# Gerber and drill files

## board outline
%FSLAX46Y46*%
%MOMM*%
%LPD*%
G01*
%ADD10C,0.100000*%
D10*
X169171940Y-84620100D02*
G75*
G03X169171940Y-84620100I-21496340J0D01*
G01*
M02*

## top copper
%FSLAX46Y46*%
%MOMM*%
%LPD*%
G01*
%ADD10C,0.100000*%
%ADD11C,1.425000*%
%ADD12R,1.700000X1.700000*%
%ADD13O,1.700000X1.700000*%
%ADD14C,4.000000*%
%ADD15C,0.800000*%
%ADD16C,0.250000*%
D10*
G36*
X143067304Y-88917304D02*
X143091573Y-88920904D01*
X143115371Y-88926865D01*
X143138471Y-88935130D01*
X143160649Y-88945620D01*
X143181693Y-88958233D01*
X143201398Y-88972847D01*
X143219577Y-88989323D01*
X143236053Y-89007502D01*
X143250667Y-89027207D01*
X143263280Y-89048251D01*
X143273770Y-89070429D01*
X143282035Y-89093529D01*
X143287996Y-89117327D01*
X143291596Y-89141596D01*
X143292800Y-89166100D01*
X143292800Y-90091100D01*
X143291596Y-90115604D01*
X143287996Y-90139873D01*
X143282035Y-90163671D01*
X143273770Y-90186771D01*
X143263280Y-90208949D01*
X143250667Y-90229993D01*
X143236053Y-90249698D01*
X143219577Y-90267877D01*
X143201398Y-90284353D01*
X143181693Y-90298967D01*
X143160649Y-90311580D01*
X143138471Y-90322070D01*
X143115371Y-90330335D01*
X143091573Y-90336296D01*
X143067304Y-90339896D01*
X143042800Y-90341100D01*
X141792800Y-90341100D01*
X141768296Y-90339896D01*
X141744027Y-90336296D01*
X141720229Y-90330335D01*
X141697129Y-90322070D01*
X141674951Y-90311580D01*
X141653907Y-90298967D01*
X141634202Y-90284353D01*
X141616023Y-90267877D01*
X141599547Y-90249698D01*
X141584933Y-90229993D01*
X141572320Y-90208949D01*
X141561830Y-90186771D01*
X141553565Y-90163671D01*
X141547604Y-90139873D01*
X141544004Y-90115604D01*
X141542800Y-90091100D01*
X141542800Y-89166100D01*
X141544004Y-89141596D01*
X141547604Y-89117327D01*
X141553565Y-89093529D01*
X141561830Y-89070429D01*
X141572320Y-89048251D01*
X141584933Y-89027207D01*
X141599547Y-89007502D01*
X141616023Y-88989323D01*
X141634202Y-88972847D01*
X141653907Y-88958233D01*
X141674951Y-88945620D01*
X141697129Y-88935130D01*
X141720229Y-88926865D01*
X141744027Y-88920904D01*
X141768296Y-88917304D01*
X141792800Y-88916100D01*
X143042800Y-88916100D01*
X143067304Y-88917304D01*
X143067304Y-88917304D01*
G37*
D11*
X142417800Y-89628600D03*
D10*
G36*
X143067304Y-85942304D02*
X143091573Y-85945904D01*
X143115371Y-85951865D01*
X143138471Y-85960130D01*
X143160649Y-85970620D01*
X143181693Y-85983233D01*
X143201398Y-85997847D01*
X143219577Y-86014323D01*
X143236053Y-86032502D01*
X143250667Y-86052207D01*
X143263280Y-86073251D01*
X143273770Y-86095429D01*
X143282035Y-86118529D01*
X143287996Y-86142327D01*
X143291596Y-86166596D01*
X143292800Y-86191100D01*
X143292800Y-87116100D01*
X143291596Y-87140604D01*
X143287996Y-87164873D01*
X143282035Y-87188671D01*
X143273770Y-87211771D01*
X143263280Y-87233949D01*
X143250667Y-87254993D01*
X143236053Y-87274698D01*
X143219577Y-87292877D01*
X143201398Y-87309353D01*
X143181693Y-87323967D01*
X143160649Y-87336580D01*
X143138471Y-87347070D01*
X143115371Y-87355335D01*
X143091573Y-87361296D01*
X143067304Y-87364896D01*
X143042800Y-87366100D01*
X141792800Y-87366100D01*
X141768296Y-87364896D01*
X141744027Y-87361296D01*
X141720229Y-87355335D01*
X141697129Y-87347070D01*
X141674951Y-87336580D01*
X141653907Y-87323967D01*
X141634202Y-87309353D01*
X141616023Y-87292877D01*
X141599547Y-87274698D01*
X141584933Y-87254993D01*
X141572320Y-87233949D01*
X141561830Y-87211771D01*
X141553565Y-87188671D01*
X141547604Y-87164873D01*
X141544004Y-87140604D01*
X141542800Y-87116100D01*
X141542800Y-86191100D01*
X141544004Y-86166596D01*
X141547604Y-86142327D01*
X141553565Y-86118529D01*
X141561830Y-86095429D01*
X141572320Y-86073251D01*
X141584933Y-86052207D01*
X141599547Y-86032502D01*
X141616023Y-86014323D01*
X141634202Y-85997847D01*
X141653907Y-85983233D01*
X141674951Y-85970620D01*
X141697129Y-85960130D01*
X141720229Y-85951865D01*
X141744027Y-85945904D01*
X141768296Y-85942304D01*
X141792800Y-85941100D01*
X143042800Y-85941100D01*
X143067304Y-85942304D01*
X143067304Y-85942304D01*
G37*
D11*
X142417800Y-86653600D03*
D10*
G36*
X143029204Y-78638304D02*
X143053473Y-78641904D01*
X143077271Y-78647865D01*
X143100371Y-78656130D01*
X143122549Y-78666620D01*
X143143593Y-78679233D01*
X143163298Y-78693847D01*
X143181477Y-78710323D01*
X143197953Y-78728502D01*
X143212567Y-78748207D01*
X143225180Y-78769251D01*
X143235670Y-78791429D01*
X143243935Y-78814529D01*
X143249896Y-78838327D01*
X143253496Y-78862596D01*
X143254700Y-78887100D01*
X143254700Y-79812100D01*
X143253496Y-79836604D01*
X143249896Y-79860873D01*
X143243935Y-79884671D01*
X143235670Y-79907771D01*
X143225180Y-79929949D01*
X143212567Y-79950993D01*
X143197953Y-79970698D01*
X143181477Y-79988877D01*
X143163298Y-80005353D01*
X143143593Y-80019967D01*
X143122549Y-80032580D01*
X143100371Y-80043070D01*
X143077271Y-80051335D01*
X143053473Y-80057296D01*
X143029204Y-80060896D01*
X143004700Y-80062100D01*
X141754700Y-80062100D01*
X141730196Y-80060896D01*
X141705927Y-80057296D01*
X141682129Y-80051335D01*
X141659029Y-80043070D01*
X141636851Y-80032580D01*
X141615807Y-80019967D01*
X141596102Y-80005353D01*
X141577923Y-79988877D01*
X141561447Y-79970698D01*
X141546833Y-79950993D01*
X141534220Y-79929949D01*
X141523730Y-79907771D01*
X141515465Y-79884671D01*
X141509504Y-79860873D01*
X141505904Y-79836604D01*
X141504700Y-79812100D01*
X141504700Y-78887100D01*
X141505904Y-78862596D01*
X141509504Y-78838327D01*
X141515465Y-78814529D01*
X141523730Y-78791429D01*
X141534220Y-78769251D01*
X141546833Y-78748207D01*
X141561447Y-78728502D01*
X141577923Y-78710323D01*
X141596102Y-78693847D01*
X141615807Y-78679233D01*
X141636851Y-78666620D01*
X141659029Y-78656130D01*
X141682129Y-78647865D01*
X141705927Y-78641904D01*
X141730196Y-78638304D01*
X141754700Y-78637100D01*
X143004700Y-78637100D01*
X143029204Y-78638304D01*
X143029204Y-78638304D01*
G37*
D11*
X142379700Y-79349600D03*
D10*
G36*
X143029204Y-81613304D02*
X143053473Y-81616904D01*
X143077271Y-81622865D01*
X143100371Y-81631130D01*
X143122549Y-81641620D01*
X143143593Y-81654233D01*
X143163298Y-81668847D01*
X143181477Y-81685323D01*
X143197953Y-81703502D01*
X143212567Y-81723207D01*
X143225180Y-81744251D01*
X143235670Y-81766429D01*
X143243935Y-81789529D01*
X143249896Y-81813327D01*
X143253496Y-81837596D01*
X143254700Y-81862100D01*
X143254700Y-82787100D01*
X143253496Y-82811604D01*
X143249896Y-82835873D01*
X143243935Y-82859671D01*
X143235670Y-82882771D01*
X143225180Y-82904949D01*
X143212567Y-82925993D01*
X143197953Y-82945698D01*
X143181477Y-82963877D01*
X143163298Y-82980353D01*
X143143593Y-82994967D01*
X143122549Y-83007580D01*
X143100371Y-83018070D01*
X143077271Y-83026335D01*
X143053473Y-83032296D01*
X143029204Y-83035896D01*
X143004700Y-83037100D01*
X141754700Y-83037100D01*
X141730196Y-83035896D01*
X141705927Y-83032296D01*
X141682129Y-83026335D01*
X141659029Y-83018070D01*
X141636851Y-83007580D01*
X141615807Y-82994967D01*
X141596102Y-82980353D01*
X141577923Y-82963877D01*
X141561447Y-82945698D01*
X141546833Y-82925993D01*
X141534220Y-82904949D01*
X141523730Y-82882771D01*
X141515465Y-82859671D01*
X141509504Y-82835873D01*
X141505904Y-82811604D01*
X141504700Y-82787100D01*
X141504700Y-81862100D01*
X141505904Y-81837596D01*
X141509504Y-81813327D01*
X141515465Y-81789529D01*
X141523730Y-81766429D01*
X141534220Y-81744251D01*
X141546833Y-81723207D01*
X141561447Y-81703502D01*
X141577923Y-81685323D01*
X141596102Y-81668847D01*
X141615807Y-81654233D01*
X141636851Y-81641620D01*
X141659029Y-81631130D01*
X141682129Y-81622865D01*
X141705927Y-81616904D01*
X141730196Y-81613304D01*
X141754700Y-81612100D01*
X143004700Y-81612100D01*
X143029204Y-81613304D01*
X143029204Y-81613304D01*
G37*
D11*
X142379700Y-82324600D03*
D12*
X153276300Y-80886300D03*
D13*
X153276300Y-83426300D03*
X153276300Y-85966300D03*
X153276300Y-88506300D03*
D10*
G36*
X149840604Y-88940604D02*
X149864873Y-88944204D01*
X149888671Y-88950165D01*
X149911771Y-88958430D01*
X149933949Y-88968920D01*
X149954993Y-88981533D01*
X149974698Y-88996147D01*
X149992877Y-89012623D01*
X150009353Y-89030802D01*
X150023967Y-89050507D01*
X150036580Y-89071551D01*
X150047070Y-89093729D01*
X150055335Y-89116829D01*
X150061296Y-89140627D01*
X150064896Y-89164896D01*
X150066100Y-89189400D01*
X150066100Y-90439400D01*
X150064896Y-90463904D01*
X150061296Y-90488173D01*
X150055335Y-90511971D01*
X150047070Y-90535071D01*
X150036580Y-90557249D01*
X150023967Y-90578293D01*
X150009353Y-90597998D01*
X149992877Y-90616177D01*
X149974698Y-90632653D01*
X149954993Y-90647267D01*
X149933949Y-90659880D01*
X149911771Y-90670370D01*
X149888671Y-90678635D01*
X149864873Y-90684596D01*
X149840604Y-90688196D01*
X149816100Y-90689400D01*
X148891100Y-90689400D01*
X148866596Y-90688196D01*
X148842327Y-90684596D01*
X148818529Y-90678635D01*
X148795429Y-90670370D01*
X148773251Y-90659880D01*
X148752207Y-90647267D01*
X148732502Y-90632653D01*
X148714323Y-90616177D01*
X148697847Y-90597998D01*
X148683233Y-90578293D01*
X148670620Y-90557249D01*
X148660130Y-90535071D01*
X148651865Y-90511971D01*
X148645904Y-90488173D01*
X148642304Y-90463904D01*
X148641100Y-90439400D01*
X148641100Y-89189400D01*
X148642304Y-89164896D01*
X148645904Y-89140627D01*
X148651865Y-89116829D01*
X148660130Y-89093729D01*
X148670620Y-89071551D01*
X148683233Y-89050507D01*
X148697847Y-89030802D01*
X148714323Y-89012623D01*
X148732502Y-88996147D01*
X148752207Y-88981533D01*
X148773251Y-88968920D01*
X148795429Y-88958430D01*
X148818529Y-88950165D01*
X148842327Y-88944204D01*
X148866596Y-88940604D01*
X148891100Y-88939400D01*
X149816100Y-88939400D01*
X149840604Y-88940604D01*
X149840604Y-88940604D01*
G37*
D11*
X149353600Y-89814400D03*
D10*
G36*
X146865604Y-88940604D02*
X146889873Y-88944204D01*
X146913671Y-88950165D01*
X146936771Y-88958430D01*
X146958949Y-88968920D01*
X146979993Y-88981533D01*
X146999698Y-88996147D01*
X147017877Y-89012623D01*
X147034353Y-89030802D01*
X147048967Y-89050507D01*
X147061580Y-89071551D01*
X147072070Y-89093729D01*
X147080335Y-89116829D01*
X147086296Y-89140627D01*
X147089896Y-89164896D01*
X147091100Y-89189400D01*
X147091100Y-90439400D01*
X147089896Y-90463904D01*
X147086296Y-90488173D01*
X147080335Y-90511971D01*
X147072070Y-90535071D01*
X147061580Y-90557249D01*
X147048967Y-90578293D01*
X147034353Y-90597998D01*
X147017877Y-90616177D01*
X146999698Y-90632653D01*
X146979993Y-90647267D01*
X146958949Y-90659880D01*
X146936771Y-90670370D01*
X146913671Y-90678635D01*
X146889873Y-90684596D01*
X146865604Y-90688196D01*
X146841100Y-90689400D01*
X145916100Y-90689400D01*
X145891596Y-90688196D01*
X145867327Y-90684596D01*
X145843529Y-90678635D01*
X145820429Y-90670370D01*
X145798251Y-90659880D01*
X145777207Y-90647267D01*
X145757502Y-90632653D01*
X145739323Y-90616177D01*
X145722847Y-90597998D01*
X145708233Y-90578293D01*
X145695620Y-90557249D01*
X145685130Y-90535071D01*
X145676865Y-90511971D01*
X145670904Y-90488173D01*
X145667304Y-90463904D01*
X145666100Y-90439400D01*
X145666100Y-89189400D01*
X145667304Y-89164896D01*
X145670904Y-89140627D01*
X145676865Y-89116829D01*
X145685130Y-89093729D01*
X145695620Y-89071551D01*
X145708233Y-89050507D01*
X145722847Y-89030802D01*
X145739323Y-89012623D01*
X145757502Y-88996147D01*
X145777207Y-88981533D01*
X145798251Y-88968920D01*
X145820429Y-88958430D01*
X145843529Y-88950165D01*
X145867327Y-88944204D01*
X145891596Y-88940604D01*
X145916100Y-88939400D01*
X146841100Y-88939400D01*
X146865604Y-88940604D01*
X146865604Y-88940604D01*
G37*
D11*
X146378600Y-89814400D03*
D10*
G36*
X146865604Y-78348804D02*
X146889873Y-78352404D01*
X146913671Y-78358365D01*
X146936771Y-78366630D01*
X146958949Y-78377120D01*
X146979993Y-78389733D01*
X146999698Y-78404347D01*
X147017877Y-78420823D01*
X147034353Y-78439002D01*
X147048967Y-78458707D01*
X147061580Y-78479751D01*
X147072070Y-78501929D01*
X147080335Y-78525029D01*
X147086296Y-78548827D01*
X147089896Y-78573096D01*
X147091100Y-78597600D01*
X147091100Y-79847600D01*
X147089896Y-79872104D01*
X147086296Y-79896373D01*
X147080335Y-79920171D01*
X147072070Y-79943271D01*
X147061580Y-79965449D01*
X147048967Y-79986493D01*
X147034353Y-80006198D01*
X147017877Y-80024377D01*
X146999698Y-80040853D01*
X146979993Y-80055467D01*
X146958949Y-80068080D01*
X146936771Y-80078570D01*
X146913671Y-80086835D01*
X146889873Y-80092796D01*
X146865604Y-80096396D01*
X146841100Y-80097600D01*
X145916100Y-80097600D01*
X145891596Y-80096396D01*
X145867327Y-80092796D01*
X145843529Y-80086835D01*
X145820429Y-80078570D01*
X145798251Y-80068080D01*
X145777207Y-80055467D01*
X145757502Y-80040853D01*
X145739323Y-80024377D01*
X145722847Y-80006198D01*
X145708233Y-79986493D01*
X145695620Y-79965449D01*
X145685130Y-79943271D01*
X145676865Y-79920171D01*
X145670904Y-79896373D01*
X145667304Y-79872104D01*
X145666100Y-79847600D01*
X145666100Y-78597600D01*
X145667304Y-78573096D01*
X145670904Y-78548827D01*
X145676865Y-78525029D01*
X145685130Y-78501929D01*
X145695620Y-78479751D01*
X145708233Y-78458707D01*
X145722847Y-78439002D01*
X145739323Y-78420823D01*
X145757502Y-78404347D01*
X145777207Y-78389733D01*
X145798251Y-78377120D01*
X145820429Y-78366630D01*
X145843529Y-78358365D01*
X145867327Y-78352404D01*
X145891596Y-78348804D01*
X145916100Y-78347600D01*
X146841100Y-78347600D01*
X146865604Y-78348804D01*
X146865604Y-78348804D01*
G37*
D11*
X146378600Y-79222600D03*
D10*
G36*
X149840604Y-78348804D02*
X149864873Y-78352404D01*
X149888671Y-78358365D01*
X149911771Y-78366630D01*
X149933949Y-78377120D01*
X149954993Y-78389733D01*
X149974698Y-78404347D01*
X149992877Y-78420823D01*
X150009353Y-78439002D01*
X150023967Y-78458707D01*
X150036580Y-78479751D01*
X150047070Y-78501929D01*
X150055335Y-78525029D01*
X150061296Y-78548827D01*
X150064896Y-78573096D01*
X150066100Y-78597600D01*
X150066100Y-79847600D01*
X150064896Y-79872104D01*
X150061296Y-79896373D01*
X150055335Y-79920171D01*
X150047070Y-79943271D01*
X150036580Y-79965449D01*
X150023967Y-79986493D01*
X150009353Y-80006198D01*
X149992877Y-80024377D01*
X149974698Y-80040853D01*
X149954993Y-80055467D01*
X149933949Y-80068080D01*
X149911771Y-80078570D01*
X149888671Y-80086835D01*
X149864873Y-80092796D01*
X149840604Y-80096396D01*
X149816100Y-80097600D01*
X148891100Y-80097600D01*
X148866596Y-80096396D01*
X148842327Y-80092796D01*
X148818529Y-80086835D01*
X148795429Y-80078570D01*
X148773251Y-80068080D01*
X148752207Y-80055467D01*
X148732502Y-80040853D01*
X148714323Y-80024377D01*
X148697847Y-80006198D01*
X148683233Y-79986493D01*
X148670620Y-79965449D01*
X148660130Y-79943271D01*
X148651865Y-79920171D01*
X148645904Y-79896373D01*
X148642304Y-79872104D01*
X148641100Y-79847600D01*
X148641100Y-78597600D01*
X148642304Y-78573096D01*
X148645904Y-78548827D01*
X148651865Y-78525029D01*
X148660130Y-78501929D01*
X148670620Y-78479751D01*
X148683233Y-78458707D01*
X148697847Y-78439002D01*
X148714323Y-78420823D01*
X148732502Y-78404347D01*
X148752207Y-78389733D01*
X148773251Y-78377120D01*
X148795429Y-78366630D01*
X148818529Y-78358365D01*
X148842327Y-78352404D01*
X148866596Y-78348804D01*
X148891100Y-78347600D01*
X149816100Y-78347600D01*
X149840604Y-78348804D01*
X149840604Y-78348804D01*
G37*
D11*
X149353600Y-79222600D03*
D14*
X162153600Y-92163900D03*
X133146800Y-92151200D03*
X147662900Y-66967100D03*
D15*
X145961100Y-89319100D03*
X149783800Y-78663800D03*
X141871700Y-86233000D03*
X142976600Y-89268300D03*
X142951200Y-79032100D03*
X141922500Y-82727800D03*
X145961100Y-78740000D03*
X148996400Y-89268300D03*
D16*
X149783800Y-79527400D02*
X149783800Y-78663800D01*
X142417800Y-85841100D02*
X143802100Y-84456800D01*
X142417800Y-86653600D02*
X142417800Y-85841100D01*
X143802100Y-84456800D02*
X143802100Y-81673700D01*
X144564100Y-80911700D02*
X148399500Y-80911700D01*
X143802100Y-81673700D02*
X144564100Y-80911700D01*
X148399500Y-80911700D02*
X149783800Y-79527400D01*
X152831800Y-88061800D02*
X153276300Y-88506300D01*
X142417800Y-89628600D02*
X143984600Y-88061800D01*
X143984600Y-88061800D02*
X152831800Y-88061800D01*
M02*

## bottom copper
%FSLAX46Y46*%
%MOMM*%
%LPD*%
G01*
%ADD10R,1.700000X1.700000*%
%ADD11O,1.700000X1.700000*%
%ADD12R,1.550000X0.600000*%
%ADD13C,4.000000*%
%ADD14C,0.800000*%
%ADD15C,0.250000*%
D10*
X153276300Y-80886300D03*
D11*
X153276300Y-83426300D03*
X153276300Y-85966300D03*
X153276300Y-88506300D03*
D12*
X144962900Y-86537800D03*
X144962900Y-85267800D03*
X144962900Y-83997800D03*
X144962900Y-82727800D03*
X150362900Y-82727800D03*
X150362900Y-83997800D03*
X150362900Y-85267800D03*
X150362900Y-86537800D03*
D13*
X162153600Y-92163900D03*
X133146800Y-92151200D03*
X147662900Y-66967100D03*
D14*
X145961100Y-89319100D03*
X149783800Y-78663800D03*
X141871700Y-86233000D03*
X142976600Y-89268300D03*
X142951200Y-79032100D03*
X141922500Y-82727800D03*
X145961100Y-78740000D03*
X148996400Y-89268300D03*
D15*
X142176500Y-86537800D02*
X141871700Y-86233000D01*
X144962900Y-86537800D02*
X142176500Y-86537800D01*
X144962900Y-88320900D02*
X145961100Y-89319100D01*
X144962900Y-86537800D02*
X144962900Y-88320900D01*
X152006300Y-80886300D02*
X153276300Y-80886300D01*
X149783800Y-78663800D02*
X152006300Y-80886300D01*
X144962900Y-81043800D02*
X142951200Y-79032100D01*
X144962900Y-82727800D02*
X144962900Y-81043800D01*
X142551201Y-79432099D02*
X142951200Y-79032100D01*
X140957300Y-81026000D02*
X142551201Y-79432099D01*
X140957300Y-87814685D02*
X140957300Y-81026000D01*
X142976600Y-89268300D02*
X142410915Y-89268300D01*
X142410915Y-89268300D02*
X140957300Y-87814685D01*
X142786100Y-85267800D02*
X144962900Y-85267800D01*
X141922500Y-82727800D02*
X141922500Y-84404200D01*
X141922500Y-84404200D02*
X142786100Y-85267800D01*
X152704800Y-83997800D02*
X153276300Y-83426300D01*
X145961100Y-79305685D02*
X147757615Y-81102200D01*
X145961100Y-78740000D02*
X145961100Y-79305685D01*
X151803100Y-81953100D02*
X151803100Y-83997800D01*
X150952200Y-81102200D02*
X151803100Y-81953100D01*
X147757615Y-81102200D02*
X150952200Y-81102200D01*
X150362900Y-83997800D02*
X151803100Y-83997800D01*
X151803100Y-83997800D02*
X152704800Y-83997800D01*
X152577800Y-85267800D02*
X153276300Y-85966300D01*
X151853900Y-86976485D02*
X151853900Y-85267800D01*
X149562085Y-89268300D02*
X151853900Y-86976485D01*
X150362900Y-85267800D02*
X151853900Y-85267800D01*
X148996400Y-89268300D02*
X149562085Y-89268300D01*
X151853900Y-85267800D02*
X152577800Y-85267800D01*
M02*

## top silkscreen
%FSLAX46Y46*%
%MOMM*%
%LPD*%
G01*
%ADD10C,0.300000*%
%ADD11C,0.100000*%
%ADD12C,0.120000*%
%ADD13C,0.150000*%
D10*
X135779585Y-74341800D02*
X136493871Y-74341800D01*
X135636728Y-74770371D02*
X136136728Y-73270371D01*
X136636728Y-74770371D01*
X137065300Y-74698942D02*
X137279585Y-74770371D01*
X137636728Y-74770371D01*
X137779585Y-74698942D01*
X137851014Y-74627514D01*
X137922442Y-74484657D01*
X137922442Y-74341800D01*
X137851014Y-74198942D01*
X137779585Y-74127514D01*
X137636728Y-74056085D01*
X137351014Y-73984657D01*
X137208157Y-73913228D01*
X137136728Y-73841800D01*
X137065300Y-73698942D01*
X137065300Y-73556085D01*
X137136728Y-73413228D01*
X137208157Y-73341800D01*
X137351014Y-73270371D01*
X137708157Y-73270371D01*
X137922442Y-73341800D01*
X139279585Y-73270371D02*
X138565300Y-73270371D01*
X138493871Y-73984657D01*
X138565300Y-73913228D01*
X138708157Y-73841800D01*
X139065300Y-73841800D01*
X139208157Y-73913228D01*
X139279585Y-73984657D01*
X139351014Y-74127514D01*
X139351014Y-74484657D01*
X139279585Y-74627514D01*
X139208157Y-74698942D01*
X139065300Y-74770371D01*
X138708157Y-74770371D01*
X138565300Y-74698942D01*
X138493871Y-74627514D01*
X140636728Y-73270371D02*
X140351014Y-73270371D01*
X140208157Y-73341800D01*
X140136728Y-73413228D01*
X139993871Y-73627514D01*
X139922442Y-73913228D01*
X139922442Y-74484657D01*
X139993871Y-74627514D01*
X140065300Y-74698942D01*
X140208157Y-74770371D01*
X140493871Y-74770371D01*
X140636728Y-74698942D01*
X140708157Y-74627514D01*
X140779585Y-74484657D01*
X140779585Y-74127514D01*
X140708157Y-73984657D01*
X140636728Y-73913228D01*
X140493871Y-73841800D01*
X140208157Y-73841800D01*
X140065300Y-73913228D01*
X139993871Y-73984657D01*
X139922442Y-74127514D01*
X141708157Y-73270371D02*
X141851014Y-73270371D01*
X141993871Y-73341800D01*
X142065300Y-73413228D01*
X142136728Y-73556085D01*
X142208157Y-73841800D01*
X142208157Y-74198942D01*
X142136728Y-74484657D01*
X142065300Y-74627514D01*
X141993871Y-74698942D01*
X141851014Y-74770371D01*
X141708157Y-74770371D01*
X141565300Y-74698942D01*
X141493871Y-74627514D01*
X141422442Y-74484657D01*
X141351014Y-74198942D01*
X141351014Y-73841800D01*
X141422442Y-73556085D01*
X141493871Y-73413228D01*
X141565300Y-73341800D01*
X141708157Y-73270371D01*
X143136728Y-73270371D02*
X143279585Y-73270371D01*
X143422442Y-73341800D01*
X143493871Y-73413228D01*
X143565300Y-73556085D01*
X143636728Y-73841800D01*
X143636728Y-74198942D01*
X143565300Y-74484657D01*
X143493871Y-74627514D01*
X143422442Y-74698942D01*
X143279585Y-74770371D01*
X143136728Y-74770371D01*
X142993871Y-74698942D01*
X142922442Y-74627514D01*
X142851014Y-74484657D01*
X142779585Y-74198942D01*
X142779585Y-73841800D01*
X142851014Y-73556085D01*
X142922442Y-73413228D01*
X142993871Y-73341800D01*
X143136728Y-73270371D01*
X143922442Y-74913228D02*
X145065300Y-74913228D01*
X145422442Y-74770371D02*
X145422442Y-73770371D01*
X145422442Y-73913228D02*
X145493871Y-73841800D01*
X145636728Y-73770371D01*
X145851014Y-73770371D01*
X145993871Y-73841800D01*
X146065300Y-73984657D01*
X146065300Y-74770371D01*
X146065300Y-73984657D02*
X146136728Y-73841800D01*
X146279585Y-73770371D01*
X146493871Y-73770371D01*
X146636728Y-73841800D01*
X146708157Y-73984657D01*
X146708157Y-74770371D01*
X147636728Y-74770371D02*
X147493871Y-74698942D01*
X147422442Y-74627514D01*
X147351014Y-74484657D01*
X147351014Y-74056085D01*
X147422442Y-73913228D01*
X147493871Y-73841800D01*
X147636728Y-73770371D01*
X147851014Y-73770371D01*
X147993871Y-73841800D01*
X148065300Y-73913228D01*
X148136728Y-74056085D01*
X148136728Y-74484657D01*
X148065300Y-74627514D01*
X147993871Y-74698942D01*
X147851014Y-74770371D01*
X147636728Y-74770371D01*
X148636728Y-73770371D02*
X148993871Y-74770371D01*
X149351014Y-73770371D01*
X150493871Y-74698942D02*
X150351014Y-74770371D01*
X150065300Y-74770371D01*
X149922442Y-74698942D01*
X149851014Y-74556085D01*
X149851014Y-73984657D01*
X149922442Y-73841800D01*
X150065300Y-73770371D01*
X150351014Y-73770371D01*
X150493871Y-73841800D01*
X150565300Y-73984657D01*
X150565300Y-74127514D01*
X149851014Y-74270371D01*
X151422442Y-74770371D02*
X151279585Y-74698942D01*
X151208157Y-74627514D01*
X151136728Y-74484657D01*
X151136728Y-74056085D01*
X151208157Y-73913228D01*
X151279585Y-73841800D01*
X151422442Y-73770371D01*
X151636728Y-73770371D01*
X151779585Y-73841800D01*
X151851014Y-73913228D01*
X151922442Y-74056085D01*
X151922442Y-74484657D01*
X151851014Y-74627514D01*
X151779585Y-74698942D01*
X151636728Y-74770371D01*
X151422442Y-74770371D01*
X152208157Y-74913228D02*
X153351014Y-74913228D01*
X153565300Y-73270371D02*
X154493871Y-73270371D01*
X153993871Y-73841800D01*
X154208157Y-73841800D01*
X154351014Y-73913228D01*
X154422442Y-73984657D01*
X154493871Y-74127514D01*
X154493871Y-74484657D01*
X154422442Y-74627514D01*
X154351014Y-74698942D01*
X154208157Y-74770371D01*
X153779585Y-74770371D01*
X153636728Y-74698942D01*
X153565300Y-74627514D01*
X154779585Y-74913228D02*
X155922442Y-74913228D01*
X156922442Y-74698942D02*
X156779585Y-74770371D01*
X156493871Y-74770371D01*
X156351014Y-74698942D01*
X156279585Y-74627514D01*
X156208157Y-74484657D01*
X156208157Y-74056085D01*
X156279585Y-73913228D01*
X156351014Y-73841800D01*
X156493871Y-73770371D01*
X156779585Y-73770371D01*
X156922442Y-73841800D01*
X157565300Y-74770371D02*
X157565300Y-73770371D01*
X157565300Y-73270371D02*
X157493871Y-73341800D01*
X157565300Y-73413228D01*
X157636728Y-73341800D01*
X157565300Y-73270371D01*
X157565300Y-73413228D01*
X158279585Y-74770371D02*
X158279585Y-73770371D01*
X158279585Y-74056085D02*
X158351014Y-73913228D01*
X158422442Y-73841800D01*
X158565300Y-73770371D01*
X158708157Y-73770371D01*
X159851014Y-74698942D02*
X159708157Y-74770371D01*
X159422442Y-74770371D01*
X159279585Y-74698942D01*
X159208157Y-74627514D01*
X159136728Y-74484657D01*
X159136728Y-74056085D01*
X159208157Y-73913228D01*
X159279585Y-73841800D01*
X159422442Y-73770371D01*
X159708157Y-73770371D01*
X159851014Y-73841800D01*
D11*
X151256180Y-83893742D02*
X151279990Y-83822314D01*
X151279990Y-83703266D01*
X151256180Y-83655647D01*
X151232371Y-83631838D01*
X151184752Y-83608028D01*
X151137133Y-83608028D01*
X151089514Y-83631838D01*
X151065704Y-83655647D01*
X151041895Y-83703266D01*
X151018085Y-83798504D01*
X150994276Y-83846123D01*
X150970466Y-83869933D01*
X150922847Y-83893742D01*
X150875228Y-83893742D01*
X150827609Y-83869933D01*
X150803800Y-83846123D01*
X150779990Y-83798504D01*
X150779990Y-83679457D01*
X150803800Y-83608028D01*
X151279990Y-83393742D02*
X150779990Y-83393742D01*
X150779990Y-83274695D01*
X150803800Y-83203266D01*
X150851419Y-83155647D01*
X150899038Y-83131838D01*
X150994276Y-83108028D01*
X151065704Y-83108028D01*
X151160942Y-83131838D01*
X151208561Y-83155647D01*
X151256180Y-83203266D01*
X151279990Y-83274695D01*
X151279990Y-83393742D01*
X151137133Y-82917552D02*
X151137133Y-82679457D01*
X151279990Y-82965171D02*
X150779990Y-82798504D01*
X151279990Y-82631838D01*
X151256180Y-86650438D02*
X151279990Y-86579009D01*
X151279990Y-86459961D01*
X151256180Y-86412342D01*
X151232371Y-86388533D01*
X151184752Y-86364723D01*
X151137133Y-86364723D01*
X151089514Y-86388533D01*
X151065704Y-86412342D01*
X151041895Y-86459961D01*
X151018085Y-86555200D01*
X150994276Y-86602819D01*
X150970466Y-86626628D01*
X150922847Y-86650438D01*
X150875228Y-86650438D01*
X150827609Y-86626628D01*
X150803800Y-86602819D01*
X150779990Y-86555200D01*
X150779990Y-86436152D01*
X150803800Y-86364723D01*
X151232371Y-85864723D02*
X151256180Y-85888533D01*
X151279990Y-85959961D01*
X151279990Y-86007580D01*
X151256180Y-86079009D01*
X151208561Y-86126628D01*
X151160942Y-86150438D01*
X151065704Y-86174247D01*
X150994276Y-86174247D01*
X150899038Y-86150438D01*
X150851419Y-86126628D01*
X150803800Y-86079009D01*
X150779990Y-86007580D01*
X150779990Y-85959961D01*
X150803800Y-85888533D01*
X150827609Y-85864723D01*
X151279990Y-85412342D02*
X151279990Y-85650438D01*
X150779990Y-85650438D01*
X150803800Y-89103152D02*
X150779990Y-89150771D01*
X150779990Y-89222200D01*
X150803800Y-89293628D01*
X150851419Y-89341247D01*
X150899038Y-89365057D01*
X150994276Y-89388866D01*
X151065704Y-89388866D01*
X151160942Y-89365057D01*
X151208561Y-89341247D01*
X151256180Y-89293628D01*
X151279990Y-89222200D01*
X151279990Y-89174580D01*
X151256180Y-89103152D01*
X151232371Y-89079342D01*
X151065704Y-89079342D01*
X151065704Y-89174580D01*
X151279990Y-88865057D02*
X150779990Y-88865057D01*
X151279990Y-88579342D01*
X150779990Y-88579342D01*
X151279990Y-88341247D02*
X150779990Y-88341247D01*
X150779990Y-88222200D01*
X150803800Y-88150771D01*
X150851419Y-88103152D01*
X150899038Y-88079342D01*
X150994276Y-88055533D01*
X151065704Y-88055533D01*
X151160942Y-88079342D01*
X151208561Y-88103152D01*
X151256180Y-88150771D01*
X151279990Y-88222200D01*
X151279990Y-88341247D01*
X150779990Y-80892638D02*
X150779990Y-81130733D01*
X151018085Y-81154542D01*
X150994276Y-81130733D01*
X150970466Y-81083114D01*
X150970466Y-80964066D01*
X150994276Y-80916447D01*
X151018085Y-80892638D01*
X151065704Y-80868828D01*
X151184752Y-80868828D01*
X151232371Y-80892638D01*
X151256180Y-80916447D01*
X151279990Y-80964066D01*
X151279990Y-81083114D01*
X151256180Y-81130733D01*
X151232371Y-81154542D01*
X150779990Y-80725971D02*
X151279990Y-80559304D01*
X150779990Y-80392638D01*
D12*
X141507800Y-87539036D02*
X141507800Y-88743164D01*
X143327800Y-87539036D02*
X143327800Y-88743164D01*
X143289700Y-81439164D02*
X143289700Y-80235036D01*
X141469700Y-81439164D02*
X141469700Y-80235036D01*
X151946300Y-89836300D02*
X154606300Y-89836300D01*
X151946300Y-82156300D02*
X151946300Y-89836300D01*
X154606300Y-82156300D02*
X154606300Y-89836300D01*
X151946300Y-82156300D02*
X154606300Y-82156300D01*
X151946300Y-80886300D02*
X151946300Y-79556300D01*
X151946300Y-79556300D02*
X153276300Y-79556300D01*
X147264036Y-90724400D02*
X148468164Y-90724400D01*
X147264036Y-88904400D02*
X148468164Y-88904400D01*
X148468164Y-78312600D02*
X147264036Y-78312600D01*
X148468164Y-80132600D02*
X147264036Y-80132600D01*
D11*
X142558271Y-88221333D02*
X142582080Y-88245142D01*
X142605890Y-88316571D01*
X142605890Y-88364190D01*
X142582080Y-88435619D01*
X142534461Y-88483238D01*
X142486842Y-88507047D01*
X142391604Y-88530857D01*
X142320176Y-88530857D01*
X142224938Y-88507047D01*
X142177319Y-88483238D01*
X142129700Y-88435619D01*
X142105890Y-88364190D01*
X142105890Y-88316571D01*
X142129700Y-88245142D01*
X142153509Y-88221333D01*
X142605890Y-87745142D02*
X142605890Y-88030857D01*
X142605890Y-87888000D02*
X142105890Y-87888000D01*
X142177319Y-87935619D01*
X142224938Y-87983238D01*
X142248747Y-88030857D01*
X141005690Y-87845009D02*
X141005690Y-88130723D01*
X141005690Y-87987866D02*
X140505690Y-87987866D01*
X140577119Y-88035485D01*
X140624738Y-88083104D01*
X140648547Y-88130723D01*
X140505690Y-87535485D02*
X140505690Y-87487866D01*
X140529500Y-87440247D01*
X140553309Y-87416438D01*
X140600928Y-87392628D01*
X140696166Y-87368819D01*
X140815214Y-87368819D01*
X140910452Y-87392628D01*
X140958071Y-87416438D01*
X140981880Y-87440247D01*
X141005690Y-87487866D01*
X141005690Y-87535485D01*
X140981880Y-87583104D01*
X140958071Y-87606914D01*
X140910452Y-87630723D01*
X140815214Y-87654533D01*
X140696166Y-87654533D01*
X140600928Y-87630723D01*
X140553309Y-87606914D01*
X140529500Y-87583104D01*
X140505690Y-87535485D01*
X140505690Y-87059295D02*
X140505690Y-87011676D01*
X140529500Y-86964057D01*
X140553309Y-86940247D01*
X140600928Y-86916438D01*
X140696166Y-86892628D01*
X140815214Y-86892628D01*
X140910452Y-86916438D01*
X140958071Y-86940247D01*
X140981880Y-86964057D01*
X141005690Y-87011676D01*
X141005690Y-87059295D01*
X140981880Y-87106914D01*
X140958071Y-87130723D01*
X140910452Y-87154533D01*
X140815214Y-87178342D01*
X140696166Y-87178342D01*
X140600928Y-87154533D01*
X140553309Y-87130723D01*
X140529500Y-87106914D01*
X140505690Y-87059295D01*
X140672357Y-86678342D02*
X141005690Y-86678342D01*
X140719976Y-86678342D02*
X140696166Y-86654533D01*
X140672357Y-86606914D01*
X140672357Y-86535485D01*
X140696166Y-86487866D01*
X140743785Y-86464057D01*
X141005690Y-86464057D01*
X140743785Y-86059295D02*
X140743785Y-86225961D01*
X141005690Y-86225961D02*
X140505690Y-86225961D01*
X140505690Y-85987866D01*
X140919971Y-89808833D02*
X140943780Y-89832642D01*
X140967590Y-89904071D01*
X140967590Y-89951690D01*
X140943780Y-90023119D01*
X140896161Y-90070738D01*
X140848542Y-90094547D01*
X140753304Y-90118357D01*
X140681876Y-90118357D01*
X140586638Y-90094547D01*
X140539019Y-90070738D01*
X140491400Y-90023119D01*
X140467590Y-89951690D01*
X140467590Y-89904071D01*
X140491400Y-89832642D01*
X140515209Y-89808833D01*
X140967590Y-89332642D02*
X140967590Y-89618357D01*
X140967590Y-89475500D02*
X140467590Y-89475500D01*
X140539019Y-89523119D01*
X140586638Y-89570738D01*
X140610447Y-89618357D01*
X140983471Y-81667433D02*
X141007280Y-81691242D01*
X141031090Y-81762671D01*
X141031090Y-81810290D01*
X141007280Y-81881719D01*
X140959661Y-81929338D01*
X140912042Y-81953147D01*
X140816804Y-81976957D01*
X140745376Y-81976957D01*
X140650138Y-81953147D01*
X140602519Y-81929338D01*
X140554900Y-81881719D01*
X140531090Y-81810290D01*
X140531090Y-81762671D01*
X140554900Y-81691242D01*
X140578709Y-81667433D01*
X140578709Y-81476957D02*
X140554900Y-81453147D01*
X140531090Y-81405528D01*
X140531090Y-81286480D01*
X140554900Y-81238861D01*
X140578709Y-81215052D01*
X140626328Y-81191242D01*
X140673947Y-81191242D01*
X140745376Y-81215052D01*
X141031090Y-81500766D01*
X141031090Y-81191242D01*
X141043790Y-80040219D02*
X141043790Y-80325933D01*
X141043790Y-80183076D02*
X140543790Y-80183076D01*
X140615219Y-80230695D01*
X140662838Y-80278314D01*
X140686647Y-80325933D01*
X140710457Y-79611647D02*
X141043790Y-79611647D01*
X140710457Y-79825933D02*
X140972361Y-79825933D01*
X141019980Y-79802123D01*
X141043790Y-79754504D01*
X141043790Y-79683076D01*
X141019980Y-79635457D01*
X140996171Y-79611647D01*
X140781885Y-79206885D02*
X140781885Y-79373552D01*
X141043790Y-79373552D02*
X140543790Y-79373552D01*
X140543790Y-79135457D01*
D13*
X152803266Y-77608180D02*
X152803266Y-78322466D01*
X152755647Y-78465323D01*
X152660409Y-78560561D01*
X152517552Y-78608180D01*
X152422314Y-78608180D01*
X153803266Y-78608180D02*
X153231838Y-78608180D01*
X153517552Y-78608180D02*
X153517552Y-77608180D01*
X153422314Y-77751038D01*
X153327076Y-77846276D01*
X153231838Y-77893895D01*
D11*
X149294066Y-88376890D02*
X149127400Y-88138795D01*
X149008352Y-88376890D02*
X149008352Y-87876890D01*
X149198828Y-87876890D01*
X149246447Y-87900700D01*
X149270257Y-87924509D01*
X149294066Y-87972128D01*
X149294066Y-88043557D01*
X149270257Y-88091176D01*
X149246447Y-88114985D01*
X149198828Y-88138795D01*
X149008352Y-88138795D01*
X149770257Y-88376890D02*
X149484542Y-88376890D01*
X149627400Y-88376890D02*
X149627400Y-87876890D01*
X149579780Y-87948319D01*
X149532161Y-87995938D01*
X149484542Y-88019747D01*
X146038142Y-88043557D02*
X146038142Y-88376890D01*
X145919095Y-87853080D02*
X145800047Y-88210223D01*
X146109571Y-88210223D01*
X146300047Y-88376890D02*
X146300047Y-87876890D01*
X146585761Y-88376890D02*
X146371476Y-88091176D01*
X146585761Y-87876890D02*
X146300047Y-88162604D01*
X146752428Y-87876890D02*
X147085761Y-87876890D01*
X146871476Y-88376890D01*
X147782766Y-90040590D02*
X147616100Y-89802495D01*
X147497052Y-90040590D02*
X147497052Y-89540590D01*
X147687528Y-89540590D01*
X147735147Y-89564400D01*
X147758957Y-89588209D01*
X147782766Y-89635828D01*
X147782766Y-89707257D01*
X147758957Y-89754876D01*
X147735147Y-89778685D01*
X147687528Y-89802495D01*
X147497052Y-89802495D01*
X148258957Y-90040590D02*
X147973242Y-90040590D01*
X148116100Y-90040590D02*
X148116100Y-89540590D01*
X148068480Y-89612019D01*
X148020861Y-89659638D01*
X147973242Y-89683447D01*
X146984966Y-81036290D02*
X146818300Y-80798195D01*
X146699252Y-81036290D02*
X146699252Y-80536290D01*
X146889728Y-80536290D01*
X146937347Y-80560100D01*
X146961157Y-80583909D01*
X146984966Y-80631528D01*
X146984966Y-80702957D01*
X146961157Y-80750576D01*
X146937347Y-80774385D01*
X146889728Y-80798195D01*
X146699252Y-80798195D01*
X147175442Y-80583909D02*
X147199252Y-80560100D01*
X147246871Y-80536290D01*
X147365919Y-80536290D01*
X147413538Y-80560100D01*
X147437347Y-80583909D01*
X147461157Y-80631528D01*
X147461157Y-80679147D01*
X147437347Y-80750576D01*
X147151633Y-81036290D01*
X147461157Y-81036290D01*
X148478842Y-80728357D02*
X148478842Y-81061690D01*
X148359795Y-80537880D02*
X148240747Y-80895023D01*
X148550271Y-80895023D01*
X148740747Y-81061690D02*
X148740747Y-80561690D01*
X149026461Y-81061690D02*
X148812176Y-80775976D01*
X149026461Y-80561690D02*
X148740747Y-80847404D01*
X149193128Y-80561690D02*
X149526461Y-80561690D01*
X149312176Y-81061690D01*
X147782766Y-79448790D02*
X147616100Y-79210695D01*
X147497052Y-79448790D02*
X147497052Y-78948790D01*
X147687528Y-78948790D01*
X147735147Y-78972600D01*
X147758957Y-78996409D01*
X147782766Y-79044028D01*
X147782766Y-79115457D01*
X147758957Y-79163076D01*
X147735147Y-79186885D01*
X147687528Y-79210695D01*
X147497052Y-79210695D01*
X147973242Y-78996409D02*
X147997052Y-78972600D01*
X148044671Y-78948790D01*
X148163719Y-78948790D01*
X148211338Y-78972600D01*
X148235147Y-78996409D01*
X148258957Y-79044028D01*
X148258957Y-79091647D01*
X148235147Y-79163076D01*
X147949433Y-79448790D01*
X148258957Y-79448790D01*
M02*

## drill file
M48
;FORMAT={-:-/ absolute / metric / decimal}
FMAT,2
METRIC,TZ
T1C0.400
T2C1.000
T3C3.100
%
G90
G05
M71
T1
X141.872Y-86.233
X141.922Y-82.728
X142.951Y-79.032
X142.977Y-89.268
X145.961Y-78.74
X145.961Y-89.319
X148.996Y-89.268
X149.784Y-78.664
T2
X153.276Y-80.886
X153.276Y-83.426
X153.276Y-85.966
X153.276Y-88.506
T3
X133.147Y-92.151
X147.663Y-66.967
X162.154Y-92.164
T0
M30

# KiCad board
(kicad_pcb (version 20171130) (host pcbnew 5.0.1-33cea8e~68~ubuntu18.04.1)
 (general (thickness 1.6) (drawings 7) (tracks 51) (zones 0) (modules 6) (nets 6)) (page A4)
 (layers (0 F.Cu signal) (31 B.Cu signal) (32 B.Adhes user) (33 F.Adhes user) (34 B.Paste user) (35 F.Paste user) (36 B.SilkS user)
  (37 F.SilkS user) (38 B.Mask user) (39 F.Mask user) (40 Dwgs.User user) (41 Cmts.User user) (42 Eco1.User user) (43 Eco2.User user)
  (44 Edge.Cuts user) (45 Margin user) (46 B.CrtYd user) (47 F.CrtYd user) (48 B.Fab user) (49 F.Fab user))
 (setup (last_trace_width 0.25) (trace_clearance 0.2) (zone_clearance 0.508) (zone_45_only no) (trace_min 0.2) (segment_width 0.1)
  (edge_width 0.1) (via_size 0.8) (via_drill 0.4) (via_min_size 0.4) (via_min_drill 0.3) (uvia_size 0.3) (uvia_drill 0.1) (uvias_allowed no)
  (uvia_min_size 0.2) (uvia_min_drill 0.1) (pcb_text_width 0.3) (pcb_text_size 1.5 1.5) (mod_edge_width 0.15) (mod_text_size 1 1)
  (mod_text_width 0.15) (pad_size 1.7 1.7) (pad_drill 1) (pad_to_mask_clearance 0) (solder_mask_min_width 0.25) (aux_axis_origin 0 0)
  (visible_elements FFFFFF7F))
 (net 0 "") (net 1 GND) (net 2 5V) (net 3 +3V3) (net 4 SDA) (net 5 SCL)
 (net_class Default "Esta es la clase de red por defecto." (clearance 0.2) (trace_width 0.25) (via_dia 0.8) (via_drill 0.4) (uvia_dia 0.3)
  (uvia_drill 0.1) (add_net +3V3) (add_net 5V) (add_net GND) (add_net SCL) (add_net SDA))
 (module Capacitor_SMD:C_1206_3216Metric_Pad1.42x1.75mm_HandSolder (layer F.Cu) (at 142.4178 88.1411 270)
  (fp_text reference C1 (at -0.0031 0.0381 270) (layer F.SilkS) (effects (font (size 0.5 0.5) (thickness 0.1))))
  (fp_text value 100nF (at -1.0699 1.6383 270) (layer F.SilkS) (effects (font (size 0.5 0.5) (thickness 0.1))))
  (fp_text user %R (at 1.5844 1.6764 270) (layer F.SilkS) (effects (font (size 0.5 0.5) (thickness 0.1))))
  (fp_line (start -0.602064 0.91) (end 0.602064 0.91) (layer F.SilkS) (width 0.12))
  (fp_line (start -0.602064 -0.91) (end 0.602064 -0.91) (layer F.SilkS) (width 0.12))
  (pad 2 smd roundrect (at 1.4875 0 270) (size 1.425 1.75) (layers F.Cu F.Paste F.Mask) (roundrect_rratio 0.175439) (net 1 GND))
  (pad 1 smd roundrect (at -1.4875 0 270) (size 1.425 1.75) (layers F.Cu F.Paste F.Mask) (roundrect_rratio 0.175439) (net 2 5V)))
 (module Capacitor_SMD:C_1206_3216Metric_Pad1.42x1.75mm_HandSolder (layer F.Cu) (at 142.3797 80.8371 90)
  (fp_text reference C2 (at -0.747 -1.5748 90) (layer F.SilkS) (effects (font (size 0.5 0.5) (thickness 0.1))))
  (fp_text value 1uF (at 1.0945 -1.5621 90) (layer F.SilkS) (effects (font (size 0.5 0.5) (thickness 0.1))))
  (fp_line (start -0.602064 0.91) (end 0.602064 0.91) (layer F.SilkS) (width 0.12))
  (fp_line (start -0.602064 -0.91) (end 0.602064 -0.91) (layer F.SilkS) (width 0.12))
  (pad 2 smd roundrect (at 1.4875 0 90) (size 1.425 1.75) (layers F.Cu F.Paste F.Mask) (roundrect_rratio 0.175439) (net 1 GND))
  (pad 1 smd roundrect (at -1.4875 0 90) (size 1.425 1.75) (layers F.Cu F.Paste F.Mask) (roundrect_rratio 0.175439) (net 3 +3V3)))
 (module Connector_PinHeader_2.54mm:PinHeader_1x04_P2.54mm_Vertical (layer F.Cu) (at 153.2763 80.8863)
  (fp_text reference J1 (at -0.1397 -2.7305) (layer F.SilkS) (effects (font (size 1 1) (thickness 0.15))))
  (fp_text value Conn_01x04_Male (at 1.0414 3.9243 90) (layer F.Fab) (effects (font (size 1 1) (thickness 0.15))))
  (fp_line (start -1.33 8.95) (end 1.33 8.95) (layer F.SilkS) (width 0.12))
  (fp_line (start -1.33 1.27) (end -1.33 8.95) (layer F.SilkS) (width 0.12))
  (fp_line (start 1.33 1.27) (end 1.33 8.95) (layer F.SilkS) (width 0.12))
  (fp_line (start -1.33 1.27) (end 1.33 1.27) (layer F.SilkS) (width 0.12))
  (fp_line (start -1.33 0) (end -1.33 -1.33) (layer F.SilkS) (width 0.12))
  (fp_line (start -1.33 -1.33) (end 0 -1.33) (layer F.SilkS) (width 0.12))
  (pad 1 thru_hole rect (at 0 0) (size 1.7 1.7) (drill 1) (layers *.Cu *.Mask) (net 2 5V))
  (pad 2 thru_hole oval (at 0 2.54) (size 1.7 1.7) (drill 1) (layers *.Cu *.Mask) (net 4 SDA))
  (pad 3 thru_hole oval (at 0 5.08) (size 1.7 1.7) (drill 1) (layers *.Cu *.Mask) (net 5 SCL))
  (pad 4 thru_hole oval (at 0 7.62) (size 1.7 1.7) (drill 1) (layers *.Cu *.Mask) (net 1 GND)))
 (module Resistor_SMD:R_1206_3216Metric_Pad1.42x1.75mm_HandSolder (layer F.Cu) (at 147.8661 89.8144)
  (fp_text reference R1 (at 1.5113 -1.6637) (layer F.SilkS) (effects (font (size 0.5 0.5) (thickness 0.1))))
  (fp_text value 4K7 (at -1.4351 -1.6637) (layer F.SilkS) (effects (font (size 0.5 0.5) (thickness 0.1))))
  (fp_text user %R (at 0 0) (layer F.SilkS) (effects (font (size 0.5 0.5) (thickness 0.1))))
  (fp_line (start -0.602064 0.91) (end 0.602064 0.91) (layer F.SilkS) (width 0.12))
  (fp_line (start -0.602064 -0.91) (end 0.602064 -0.91) (layer F.SilkS) (width 0.12))
  (pad 2 smd roundrect (at 1.4875 0) (size 1.425 1.75) (layers F.Cu F.Paste F.Mask) (roundrect_rratio 0.175439) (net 5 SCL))
  (pad 1 smd roundrect (at -1.4875 0) (size 1.425 1.75) (layers F.Cu F.Paste F.Mask) (roundrect_rratio 0.175439) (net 2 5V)))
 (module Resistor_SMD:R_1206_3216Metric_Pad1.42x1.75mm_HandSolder (layer F.Cu) (at 147.8661 79.2226 180)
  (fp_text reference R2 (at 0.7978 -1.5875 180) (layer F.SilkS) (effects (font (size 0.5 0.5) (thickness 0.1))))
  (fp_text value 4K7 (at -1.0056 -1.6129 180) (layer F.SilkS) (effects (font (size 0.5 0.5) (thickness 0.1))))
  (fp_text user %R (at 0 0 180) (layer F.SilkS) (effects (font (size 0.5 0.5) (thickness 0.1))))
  (fp_line (start -0.602064 0.91) (end 0.602064 0.91) (layer F.SilkS) (width 0.12))
  (fp_line (start -0.602064 -0.91) (end 0.602064 -0.91) (layer F.SilkS) (width 0.12))
  (pad 2 smd roundrect (at 1.4875 0 180) (size 1.425 1.75) (layers F.Cu F.Paste F.Mask) (roundrect_rratio 0.175439) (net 4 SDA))
  (pad 1 smd roundrect (at -1.4875 0 180) (size 1.425 1.75) (layers F.Cu F.Paste F.Mask) (roundrect_rratio 0.175439) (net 2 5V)))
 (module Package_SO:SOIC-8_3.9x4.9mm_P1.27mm (layer B.Cu) (at 147.6629 84.6328)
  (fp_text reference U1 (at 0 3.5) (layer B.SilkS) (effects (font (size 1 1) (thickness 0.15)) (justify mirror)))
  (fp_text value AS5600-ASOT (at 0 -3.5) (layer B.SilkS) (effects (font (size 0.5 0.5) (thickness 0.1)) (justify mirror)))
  (pad 1 smd rect (at -2.7 1.905) (size 1.55 0.6) (layers B.Cu B.Paste B.Mask) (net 2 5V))
  (pad 2 smd rect (at -2.7 0.635) (size 1.55 0.6) (layers B.Cu B.Paste B.Mask) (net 3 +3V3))
  (pad 3 smd rect (at -2.7 -0.635) (size 1.55 0.6) (layers B.Cu B.Paste B.Mask))
  (pad 4 smd rect (at -2.7 -1.905) (size 1.55 0.6) (layers B.Cu B.Paste B.Mask) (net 1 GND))
  (pad 5 smd rect (at 2.7 -1.905) (size 1.55 0.6) (layers B.Cu B.Paste B.Mask))
  (pad 6 smd rect (at 2.7 -0.635) (size 1.55 0.6) (layers B.Cu B.Paste B.Mask) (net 4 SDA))
  (pad 7 smd rect (at 2.7 0.635) (size 1.55 0.6) (layers B.Cu B.Paste B.Mask) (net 5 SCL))
  (pad 8 smd rect (at 2.7 1.905) (size 1.55 0.6) (layers B.Cu B.Paste B.Mask)))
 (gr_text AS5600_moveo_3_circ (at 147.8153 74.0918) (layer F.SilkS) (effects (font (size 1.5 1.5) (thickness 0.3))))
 (gr_circle (center 147.6756 84.6201) (end 169.17194 84.6201) (layer Edge.Cuts) (width 0.1))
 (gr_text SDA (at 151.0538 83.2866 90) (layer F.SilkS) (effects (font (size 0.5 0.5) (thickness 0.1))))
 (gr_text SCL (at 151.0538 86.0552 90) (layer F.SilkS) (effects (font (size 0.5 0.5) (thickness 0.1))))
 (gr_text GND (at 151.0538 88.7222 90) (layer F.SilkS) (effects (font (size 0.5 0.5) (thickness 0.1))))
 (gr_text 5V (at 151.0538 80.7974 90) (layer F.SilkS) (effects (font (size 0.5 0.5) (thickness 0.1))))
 (via (at 162.1536 92.1639) (size 4) (drill 3.1) (layers F.Cu B.Cu) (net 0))
 (via (at 133.1468 92.1512) (size 4) (drill 3.1) (layers F.Cu B.Cu) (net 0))
 (via (at 147.6629 66.9671) (size 4) (drill 3.1) (layers F.Cu B.Cu) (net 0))
 (via (at 145.9611 89.3191) (size 0.8) (drill 0.4) (layers F.Cu B.Cu) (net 2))
 (via (at 149.7838 78.6638) (size 0.8) (drill 0.4) (layers F.Cu B.Cu) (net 2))
 (via (at 141.8717 86.233) (size 0.8) (drill 0.4) (layers F.Cu B.Cu) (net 2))
 (segment (start 142.1765 86.5378) (end 141.8717 86.233) (width 0.25) (layer B.Cu) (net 2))
 (segment (start 144.9629 86.5378) (end 142.1765 86.5378) (width 0.25) (layer B.Cu) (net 2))
 (segment (start 144.9629 88.3209) (end 145.9611 89.3191) (width 0.25) (layer B.Cu) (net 2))
 (segment (start 144.9629 86.5378) (end 144.9629 88.3209) (width 0.25) (layer B.Cu) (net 2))
 (segment (start 152.0063 80.8863) (end 153.2763 80.8863) (width 0.25) (layer B.Cu) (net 2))
 (segment (start 149.7838 78.6638) (end 152.0063 80.8863) (width 0.25) (layer B.Cu) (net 2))
 (segment (start 149.7838 79.5274) (end 149.7838 78.6638) (width 0.25) (layer F.Cu) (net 2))
 (segment (start 142.4178 85.8411) (end 143.8021 84.4568) (width 0.25) (layer F.Cu) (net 2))
 (segment (start 142.4178 86.6536) (end 142.4178 85.8411) (width 0.25) (layer F.Cu) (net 2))
 (segment (start 143.8021 84.4568) (end 143.8021 81.6737) (width 0.25) (layer F.Cu) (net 2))
 (segment (start 144.5641 80.9117) (end 148.3995 80.9117) (width 0.25) (layer F.Cu) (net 2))
 (segment (start 143.8021 81.6737) (end 144.5641 80.9117) (width 0.25) (layer F.Cu) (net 2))
 (segment (start 148.3995 80.9117) (end 149.7838 79.5274) (width 0.25) (layer F.Cu) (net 2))
 (via (at 142.9766 89.2683) (size 0.8) (drill 0.4) (layers F.Cu B.Cu) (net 1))
 (via (at 142.9512 79.0321) (size 0.8) (drill 0.4) (layers F.Cu B.Cu) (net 1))
 (segment (start 144.9629 81.0438) (end 142.9512 79.0321) (width 0.25) (layer B.Cu) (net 1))
 (segment (start 144.9629 82.7278) (end 144.9629 81.0438) (width 0.25) (layer B.Cu) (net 1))
 (segment (start 152.8318 88.0618) (end 153.2763 88.5063) (width 0.25) (layer F.Cu) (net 1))
 (segment (start 142.4178 89.6286) (end 143.9846 88.0618) (width 0.25) (layer F.Cu) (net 1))
 (segment (start 143.9846 88.0618) (end 152.8318 88.0618) (width 0.25) (layer F.Cu) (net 1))
 (segment (start 142.551201 79.432099) (end 142.9512 79.0321) (width 0.25) (layer B.Cu) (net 1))
 (segment (start 140.9573 81.026) (end 142.551201 79.432099) (width 0.25) (layer B.Cu) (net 1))
 (segment (start 140.9573 87.814685) (end 140.9573 81.026) (width 0.25) (layer B.Cu) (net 1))
 (segment (start 142.9766 89.2683) (end 142.410915 89.2683) (width 0.25) (layer B.Cu) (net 1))
 (segment (start 142.410915 89.2683) (end 140.9573 87.814685) (width 0.25) (layer B.Cu) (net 1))
 (via (at 141.9225 82.7278) (size 0.8) (drill 0.4) (layers F.Cu B.Cu) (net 3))
 (segment (start 142.7861 85.2678) (end 144.9629 85.2678) (width 0.25) (layer B.Cu) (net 3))
 (segment (start 141.9225 82.7278) (end 141.9225 84.4042) (width 0.25) (layer B.Cu) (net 3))
 (segment (start 141.9225 84.4042) (end 142.7861 85.2678) (width 0.25) (layer B.Cu) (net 3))
 (via (at 145.9611 78.74) (size 0.8) (drill 0.4) (layers F.Cu B.Cu) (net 4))
 (segment (start 152.7048 83.9978) (end 153.2763 83.4263) (width 0.25) (layer B.Cu) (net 4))
 (segment (start 145.9611 79.305685) (end 147.757615 81.1022) (width 0.25) (layer B.Cu) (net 4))
 (segment (start 145.9611 78.74) (end 145.9611 79.305685) (width 0.25) (layer B.Cu) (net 4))
 (segment (start 151.8031 81.9531) (end 151.8031 83.9978) (width 0.25) (layer B.Cu) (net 4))
 (segment (start 150.9522 81.1022) (end 151.8031 81.9531) (width 0.25) (layer B.Cu) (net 4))
 (segment (start 147.757615 81.1022) (end 150.9522 81.1022) (width 0.25) (layer B.Cu) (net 4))
 (segment (start 150.3629 83.9978) (end 151.8031 83.9978) (width 0.25) (layer B.Cu) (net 4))
 (segment (start 151.8031 83.9978) (end 152.7048 83.9978) (width 0.25) (layer B.Cu) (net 4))
 (via (at 148.9964 89.2683) (size 0.8) (drill 0.4) (layers F.Cu B.Cu) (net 5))
 (segment (start 152.5778 85.2678) (end 153.2763 85.9663) (width 0.25) (layer B.Cu) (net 5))
 (segment (start 151.8539 86.976485) (end 151.8539 85.2678) (width 0.25) (layer B.Cu) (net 5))
 (segment (start 149.562085 89.2683) (end 151.8539 86.976485) (width 0.25) (layer B.Cu) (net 5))
 (segment (start 150.3629 85.2678) (end 151.8539 85.2678) (width 0.25) (layer B.Cu) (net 5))
 (segment (start 148.9964 89.2683) (end 149.562085 89.2683) (width 0.25) (layer B.Cu) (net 5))
 (segment (start 151.8539 85.2678) (end 152.5778 85.2678) (width 0.25) (layer B.Cu) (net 5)))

